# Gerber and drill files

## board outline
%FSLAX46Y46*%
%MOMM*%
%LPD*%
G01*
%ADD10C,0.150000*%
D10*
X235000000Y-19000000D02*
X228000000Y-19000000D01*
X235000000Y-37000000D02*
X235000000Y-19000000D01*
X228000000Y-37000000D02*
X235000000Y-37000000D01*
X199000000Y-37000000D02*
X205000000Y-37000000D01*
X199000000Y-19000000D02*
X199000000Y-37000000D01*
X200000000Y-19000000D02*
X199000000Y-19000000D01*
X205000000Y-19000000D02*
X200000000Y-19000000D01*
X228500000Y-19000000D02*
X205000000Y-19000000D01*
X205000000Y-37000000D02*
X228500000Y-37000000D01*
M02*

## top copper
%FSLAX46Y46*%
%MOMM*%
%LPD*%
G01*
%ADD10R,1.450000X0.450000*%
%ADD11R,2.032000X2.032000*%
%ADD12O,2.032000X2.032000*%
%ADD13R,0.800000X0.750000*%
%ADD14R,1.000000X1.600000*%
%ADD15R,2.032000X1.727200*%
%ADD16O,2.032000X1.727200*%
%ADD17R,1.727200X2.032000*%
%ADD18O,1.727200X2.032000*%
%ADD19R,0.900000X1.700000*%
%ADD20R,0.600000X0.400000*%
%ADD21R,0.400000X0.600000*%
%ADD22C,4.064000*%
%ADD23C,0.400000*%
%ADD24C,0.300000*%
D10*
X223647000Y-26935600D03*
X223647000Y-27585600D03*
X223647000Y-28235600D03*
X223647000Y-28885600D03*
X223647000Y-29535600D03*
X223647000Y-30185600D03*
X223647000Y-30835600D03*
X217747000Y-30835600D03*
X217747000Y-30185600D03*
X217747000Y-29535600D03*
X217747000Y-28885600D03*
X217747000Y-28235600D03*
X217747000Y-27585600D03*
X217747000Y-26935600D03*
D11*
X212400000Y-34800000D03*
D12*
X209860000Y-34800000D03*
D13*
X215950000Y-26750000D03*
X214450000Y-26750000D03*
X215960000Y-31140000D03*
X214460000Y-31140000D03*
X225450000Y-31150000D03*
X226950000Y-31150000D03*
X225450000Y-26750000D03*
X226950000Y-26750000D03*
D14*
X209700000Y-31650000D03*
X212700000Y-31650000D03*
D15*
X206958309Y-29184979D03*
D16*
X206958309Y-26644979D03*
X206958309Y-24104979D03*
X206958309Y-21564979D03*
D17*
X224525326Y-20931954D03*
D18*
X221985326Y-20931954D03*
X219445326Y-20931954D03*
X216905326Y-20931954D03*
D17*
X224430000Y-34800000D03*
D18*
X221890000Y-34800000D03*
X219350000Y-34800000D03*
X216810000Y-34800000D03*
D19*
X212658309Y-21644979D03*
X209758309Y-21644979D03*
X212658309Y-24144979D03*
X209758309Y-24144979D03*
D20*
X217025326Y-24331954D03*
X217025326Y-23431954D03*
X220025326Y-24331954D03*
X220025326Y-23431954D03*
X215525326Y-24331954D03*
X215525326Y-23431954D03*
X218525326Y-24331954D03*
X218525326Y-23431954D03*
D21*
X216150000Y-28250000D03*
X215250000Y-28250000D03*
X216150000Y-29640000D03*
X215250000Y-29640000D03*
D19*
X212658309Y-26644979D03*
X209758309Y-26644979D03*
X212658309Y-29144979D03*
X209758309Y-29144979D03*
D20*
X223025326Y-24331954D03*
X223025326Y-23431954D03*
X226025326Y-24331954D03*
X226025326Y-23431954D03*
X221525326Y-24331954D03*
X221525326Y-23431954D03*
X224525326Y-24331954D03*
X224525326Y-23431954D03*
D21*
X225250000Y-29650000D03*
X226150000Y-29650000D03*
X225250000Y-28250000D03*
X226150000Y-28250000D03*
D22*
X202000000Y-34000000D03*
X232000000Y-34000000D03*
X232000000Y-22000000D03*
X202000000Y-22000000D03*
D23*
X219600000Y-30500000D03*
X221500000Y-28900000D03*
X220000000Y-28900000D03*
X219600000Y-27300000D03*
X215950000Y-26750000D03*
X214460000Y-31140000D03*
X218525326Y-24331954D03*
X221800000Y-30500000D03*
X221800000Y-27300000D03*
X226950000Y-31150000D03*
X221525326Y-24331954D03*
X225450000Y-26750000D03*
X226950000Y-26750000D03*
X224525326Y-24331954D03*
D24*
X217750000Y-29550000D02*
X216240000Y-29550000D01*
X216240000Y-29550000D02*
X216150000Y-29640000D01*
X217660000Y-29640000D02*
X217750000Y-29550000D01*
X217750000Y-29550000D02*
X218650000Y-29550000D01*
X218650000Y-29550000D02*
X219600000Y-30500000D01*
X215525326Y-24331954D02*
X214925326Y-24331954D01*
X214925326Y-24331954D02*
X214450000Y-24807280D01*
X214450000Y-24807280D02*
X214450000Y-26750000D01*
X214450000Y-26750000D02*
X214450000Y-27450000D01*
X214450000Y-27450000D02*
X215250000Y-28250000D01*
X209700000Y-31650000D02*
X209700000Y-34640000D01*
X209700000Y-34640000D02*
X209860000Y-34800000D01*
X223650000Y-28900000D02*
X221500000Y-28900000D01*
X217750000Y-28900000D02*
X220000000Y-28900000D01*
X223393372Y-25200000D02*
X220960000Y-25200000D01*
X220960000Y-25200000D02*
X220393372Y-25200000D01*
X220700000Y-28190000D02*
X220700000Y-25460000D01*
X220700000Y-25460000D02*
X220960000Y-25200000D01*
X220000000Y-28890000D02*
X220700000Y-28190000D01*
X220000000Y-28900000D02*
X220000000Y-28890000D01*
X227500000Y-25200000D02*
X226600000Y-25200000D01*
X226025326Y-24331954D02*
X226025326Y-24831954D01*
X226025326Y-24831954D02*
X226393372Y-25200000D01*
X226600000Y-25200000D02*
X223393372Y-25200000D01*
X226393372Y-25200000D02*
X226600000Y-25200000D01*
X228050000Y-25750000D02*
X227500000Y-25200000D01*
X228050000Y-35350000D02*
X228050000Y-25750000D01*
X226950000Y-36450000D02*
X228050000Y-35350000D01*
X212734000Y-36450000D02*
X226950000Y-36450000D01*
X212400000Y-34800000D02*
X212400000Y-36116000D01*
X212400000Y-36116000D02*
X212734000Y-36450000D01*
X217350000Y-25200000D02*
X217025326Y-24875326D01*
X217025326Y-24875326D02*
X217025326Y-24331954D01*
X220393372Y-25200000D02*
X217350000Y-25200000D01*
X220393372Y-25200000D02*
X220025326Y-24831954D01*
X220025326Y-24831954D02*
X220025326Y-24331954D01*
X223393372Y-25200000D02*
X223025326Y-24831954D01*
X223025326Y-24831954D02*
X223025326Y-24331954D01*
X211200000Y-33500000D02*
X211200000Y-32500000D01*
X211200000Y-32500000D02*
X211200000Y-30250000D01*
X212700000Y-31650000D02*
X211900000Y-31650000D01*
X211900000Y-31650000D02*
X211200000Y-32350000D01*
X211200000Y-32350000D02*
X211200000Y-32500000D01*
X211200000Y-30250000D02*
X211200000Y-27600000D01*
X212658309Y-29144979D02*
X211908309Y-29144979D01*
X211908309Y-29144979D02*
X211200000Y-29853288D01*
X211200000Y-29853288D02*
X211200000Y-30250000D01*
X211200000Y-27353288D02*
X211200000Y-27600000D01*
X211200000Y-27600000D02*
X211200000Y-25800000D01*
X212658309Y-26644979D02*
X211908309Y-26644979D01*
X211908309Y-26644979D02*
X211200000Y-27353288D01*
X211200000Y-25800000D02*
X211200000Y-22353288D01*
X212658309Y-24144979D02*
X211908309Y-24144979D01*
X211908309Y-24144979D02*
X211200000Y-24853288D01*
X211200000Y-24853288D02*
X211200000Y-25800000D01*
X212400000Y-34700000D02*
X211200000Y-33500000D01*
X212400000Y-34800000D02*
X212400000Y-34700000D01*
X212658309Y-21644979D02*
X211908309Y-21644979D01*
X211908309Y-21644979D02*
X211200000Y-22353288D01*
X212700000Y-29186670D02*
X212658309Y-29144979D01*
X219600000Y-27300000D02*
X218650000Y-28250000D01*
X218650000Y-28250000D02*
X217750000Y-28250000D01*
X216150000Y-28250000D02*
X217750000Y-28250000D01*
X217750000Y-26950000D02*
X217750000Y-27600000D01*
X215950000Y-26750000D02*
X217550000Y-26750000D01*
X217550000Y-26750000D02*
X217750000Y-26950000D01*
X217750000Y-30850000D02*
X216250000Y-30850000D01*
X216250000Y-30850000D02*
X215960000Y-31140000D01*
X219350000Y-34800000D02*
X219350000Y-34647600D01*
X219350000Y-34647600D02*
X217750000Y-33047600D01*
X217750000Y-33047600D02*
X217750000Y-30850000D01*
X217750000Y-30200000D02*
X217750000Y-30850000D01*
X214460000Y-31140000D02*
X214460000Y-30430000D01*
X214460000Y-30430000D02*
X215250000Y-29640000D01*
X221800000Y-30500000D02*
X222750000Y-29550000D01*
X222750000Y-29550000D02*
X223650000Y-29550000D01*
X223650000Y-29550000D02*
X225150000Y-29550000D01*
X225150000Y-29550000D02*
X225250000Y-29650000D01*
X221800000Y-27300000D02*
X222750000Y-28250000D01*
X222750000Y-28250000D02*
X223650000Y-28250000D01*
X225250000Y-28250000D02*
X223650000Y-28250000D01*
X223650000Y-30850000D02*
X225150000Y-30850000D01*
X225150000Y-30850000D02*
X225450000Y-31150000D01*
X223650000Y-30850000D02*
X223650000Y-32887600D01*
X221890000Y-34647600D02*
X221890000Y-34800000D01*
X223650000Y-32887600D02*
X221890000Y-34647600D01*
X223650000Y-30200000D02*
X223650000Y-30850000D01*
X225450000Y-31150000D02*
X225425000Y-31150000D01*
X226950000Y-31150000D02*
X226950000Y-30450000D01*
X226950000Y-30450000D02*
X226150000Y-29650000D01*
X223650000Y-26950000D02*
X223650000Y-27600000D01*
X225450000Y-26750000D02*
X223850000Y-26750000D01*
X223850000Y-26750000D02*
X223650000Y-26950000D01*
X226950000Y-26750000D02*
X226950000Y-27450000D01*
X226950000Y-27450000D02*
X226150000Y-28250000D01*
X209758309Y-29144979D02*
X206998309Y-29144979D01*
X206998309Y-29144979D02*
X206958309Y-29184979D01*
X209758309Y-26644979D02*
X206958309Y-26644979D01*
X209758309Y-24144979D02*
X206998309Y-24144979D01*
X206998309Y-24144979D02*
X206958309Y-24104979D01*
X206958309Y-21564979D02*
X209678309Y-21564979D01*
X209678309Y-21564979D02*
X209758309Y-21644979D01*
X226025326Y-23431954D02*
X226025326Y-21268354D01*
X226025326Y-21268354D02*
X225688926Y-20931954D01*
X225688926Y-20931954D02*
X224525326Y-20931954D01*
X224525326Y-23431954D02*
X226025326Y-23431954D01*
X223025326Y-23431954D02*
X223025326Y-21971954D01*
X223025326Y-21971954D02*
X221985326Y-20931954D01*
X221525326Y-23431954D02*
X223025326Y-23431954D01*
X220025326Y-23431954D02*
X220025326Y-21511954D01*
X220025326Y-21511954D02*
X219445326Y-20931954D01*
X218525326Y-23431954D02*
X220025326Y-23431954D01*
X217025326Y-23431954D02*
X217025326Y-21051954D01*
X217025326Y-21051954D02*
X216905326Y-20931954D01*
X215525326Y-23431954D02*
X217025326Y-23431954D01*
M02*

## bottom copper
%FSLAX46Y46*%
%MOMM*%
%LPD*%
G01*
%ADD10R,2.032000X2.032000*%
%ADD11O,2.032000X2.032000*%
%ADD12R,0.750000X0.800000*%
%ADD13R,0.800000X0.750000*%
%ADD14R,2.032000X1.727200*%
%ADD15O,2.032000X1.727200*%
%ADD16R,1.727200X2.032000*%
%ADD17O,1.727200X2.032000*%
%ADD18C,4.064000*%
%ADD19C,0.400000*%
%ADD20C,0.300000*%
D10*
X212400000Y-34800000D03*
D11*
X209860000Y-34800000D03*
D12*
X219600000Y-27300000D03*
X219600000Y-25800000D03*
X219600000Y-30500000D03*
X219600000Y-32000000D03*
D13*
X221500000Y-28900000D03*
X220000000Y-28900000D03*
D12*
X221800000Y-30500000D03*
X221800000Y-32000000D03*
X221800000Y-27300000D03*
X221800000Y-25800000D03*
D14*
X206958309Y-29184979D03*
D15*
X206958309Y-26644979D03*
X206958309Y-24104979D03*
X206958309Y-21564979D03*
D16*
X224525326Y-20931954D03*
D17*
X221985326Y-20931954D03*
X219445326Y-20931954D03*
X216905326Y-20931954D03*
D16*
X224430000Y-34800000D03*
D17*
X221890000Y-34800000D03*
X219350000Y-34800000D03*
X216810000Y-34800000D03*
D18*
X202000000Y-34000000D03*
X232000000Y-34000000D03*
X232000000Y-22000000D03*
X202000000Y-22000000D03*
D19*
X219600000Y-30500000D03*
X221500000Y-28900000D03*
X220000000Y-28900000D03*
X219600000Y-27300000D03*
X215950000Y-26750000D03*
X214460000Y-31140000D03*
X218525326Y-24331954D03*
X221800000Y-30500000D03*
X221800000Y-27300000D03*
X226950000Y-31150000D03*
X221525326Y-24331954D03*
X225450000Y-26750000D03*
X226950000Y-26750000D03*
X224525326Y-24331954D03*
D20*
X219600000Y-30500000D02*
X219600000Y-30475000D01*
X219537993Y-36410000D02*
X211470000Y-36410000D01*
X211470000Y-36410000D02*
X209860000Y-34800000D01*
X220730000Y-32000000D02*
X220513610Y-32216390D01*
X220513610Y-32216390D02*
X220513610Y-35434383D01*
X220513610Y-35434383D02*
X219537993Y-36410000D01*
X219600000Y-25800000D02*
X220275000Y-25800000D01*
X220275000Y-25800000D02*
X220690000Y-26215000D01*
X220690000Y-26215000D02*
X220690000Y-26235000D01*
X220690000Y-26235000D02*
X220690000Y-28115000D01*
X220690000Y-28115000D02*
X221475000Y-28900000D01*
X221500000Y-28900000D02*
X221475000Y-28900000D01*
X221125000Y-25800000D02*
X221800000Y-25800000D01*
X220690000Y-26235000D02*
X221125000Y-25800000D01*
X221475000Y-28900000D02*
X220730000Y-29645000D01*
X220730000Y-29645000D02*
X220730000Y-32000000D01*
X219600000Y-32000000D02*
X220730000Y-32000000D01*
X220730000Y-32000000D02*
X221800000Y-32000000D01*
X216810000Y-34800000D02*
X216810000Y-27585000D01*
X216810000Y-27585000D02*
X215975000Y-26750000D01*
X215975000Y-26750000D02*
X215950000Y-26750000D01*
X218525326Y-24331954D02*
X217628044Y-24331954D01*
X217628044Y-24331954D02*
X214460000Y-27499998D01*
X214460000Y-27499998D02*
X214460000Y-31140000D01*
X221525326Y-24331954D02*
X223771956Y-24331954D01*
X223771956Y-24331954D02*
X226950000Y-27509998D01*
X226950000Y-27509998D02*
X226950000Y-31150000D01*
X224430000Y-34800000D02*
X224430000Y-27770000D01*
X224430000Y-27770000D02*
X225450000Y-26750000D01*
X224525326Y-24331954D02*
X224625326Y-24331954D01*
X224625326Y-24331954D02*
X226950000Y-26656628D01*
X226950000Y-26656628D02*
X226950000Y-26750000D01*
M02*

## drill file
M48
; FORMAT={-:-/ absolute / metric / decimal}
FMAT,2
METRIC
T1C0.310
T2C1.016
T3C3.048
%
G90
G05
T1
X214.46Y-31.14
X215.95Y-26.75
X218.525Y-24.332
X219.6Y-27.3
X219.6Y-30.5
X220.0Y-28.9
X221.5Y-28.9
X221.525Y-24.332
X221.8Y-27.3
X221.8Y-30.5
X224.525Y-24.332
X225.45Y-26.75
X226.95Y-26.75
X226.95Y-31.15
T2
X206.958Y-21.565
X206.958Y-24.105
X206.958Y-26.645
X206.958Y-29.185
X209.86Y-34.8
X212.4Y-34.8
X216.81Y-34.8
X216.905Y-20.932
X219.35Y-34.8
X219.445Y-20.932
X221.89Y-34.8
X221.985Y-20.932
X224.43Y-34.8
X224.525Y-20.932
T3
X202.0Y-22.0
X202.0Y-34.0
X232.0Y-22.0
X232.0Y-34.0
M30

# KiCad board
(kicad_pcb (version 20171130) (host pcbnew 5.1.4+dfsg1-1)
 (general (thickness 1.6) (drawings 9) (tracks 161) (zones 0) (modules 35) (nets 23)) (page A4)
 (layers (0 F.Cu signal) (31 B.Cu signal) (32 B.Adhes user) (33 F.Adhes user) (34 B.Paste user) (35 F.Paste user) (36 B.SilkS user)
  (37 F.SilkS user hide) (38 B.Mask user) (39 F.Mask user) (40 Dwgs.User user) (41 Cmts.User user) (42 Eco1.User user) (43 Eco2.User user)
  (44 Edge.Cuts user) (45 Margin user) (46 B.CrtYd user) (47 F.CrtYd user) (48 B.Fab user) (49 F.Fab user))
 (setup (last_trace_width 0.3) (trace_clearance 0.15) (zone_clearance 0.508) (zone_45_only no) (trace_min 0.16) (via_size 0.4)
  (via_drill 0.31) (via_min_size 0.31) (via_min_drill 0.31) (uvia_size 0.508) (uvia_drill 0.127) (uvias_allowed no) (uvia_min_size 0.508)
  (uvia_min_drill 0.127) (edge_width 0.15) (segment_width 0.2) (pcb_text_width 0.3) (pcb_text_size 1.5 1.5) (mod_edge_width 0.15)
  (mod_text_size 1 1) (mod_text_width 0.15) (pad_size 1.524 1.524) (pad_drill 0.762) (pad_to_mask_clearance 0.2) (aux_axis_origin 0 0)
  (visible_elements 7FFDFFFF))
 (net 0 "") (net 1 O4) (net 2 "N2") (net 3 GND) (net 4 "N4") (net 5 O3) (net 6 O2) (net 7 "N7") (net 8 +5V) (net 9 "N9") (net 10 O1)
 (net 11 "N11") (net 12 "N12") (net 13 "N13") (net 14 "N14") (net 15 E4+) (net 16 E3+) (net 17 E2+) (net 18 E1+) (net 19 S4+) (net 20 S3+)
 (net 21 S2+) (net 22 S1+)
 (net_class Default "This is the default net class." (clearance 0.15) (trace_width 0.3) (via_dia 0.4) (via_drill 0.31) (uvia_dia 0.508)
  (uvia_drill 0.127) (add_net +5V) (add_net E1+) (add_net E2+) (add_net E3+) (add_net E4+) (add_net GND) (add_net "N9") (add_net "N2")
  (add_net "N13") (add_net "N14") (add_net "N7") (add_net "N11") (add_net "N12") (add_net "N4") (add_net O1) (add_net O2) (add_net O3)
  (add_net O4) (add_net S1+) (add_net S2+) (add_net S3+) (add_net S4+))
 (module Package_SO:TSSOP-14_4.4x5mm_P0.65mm (layer F.Cu) (at 220.697 28.8856)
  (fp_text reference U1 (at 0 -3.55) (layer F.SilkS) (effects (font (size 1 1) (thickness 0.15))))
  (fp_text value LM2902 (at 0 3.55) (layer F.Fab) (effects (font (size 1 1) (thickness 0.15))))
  (pad 14 smd rect (at 2.95 -1.95) (size 1.45 0.45) (layers F.Cu F.Paste F.Mask) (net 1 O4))
  (pad 13 smd rect (at 2.95 -1.3) (size 1.45 0.45) (layers F.Cu F.Paste F.Mask) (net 1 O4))
  (pad 12 smd rect (at 2.95 -0.65) (size 1.45 0.45) (layers F.Cu F.Paste F.Mask) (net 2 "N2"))
  (pad 11 smd rect (at 2.95 0) (size 1.45 0.45) (layers F.Cu F.Paste F.Mask) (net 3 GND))
  (pad 10 smd rect (at 2.95 0.65) (size 1.45 0.45) (layers F.Cu F.Paste F.Mask) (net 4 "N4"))
  (pad 9 smd rect (at 2.95 1.3) (size 1.45 0.45) (layers F.Cu F.Paste F.Mask) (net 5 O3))
  (pad 8 smd rect (at 2.95 1.95) (size 1.45 0.45) (layers F.Cu F.Paste F.Mask) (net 5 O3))
  (pad 7 smd rect (at -2.95 1.95) (size 1.45 0.45) (layers F.Cu F.Paste F.Mask) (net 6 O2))
  (pad 6 smd rect (at -2.95 1.3) (size 1.45 0.45) (layers F.Cu F.Paste F.Mask) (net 6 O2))
  (pad 5 smd rect (at -2.95 0.65) (size 1.45 0.45) (layers F.Cu F.Paste F.Mask) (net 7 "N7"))
  (pad 4 smd rect (at -2.95 0) (size 1.45 0.45) (layers F.Cu F.Paste F.Mask) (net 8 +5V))
  (pad 3 smd rect (at -2.95 -0.65) (size 1.45 0.45) (layers F.Cu F.Paste F.Mask) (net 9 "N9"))
  (pad 2 smd rect (at -2.95 -1.3) (size 1.45 0.45) (layers F.Cu F.Paste F.Mask) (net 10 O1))
  (pad 1 smd rect (at -2.95 -1.95) (size 1.45 0.45) (layers F.Cu F.Paste F.Mask) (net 10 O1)))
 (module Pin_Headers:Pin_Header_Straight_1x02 (layer F.Cu) (at 212.4 34.8 270)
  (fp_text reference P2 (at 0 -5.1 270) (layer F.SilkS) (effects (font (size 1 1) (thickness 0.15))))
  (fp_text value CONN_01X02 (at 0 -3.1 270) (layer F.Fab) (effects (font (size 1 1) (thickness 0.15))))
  (pad 1 thru_hole rect (at 0 0 270) (size 2.032 2.032) (drill 1.016) (layers *.Cu *.Mask F.SilkS) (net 8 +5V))
  (pad 2 thru_hole oval (at 0 2.54 270) (size 2.032 2.032) (drill 1.016) (layers *.Cu *.Mask F.SilkS) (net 3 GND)))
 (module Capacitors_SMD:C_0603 (layer B.Cu) (at 219.6 26.55 90)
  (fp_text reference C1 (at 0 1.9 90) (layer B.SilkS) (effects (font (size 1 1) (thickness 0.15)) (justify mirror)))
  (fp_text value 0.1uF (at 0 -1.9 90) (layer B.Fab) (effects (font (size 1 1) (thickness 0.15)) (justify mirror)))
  (pad 1 smd rect (at -0.75 0 90) (size 0.8 0.75) (layers B.Cu B.Paste B.Mask) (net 9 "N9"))
  (pad 2 smd rect (at 0.75 0 90) (size 0.8 0.75) (layers B.Cu B.Paste B.Mask) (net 3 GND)))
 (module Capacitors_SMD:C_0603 (layer B.Cu) (at 219.6 31.25 270)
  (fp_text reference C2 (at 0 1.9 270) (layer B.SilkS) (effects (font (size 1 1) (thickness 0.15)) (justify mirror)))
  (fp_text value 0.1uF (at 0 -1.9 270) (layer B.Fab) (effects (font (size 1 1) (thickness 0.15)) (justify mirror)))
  (pad 1 smd rect (at -0.75 0 270) (size 0.8 0.75) (layers B.Cu B.Paste B.Mask) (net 7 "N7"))
  (pad 2 smd rect (at 0.75 0 270) (size 0.8 0.75) (layers B.Cu B.Paste B.Mask) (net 3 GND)))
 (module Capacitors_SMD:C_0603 (layer F.Cu) (at 215.2 26.75 180)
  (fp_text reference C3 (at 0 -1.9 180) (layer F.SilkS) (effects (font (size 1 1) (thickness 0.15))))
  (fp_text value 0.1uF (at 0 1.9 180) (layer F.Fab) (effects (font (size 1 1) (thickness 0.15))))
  (pad 1 smd rect (at -0.75 0 180) (size 0.8 0.75) (layers F.Cu F.Paste F.Mask) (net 10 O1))
  (pad 2 smd rect (at 0.75 0 180) (size 0.8 0.75) (layers F.Cu F.Paste F.Mask) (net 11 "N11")))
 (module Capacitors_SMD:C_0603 (layer F.Cu) (at 215.21 31.14 180)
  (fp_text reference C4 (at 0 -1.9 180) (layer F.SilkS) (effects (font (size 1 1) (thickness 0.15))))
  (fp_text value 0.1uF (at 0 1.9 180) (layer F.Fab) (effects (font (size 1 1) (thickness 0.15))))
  (pad 1 smd rect (at -0.75 0 180) (size 0.8 0.75) (layers F.Cu F.Paste F.Mask) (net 6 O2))
  (pad 2 smd rect (at 0.75 0 180) (size 0.8 0.75) (layers F.Cu F.Paste F.Mask) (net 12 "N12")))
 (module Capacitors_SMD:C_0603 (layer B.Cu) (at 220.75 28.9 180)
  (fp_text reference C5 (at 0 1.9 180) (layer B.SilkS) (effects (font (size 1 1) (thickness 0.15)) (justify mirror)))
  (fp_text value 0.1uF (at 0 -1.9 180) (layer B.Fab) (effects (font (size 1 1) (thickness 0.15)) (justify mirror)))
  (pad 1 smd rect (at -0.75 0 180) (size 0.8 0.75) (layers B.Cu B.Paste B.Mask) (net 3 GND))
  (pad 2 smd rect (at 0.75 0 180) (size 0.8 0.75) (layers B.Cu B.Paste B.Mask) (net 8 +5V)))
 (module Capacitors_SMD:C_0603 (layer B.Cu) (at 221.8 31.25 270)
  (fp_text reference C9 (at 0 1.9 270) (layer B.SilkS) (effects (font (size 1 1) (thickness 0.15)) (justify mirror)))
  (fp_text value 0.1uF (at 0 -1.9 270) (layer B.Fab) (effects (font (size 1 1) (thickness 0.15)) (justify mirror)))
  (pad 1 smd rect (at -0.75 0 270) (size 0.8 0.75) (layers B.Cu B.Paste B.Mask) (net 4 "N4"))
  (pad 2 smd rect (at 0.75 0 270) (size 0.8 0.75) (layers B.Cu B.Paste B.Mask) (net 3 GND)))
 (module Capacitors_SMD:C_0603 (layer B.Cu) (at 221.8 26.55 90)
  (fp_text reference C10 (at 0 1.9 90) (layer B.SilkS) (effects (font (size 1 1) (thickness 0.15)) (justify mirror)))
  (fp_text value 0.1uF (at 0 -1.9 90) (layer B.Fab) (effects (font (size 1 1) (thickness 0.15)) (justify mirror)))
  (pad 1 smd rect (at -0.75 0 90) (size 0.8 0.75) (layers B.Cu B.Paste B.Mask) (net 2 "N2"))
  (pad 2 smd rect (at 0.75 0 90) (size 0.8 0.75) (layers B.Cu B.Paste B.Mask) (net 3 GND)))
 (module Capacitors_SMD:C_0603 (layer F.Cu) (at 226.2 31.15)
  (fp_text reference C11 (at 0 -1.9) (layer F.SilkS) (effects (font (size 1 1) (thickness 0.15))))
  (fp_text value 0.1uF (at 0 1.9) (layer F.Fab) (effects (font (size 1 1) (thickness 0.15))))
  (pad 1 smd rect (at -0.75 0) (size 0.8 0.75) (layers F.Cu F.Paste F.Mask) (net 5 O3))
  (pad 2 smd rect (at 0.75 0) (size 0.8 0.75) (layers F.Cu F.Paste F.Mask) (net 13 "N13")))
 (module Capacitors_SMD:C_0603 (layer F.Cu) (at 226.2 26.75)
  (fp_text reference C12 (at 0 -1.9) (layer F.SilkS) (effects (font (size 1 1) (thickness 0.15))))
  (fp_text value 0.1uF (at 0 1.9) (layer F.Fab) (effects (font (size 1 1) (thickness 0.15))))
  (pad 1 smd rect (at -0.75 0) (size 0.8 0.75) (layers F.Cu F.Paste F.Mask) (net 1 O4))
  (pad 2 smd rect (at 0.75 0) (size 0.8 0.75) (layers F.Cu F.Paste F.Mask) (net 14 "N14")))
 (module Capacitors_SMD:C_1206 (layer F.Cu) (at 211.2 31.65)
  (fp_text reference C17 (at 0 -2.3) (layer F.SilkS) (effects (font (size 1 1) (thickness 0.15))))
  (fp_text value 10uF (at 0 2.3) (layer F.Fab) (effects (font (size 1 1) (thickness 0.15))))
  (pad 1 smd rect (at -1.5 0) (size 1 1.6) (layers F.Cu F.Paste F.Mask) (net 3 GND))
  (pad 2 smd rect (at 1.5 0) (size 1 1.6) (layers F.Cu F.Paste F.Mask) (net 8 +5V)))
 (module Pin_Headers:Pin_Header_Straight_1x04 (layer F.Cu) (at 206.958309 29.184979 180)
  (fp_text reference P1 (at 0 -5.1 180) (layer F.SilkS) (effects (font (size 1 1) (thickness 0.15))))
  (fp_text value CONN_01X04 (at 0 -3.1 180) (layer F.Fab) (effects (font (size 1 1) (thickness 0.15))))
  (pad 1 thru_hole rect (at 0 0 180) (size 2.032 1.7272) (drill 1.016) (layers *.Cu *.Mask F.SilkS) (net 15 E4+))
  (pad 2 thru_hole oval (at 0 2.54 180) (size 2.032 1.7272) (drill 1.016) (layers *.Cu *.Mask F.SilkS) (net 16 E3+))
  (pad 3 thru_hole oval (at 0 5.08 180) (size 2.032 1.7272) (drill 1.016) (layers *.Cu *.Mask F.SilkS) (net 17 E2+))
  (pad 4 thru_hole oval (at 0 7.62 180) (size 2.032 1.7272) (drill 1.016) (layers *.Cu *.Mask F.SilkS) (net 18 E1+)))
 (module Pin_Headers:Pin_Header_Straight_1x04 (layer F.Cu) (at 224.525326 20.931954 270)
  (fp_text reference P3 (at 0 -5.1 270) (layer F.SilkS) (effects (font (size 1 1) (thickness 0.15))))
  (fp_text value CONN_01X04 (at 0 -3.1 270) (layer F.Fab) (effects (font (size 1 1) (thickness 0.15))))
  (pad 1 thru_hole rect (at 0 0 270) (size 2.032 1.7272) (drill 1.016) (layers *.Cu *.Mask F.SilkS) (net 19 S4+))
  (pad 2 thru_hole oval (at 0 2.54 270) (size 2.032 1.7272) (drill 1.016) (layers *.Cu *.Mask F.SilkS) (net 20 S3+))
  (pad 3 thru_hole oval (at 0 5.08 270) (size 2.032 1.7272) (drill 1.016) (layers *.Cu *.Mask F.SilkS) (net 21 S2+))
  (pad 4 thru_hole oval (at 0 7.62 270) (size 2.032 1.7272) (drill 1.016) (layers *.Cu *.Mask F.SilkS) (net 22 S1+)))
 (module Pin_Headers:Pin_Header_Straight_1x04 (layer F.Cu) (at 224.43 34.8 270)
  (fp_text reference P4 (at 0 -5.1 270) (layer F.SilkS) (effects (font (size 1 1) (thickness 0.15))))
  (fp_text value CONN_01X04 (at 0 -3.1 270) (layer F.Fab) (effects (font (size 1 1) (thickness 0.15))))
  (pad 1 thru_hole rect (at 0 0 270) (size 2.032 1.7272) (drill 1.016) (layers *.Cu *.Mask F.SilkS) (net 1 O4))
  (pad 2 thru_hole oval (at 0 2.54 270) (size 2.032 1.7272) (drill 1.016) (layers *.Cu *.Mask F.SilkS) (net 5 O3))
  (pad 3 thru_hole oval (at 0 5.08 270) (size 2.032 1.7272) (drill 1.016) (layers *.Cu *.Mask F.SilkS) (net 6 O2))
  (pad 4 thru_hole oval (at 0 7.62 270) (size 2.032 1.7272) (drill 1.016) (layers *.Cu *.Mask F.SilkS) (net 10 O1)))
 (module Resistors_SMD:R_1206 (layer F.Cu) (at 211.208309 21.644979 180)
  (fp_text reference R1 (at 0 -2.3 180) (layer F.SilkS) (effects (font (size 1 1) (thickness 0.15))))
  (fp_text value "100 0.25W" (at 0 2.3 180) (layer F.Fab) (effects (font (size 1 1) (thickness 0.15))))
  (pad 1 smd rect (at -1.45 0 180) (size 0.9 1.7) (layers F.Cu F.Paste F.Mask) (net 8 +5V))
  (pad 2 smd rect (at 1.45 0 180) (size 0.9 1.7) (layers F.Cu F.Paste F.Mask) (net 18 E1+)))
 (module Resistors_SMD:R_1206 (layer F.Cu) (at 211.208309 24.144979 180)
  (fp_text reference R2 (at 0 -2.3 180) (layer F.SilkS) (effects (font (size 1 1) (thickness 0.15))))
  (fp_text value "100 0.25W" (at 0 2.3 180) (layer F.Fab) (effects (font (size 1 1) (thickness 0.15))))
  (pad 1 smd rect (at -1.45 0 180) (size 0.9 1.7) (layers F.Cu F.Paste F.Mask) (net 8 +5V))
  (pad 2 smd rect (at 1.45 0 180) (size 0.9 1.7) (layers F.Cu F.Paste F.Mask) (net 17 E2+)))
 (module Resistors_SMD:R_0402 (layer F.Cu) (at 217.025326 23.881954 90)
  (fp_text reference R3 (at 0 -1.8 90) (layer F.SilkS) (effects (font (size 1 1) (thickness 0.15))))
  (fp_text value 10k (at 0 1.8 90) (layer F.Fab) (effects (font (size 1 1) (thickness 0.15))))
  (pad 1 smd rect (at -0.45 0 90) (size 0.4 0.6) (layers F.Cu F.Paste F.Mask) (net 8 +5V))
  (pad 2 smd rect (at 0.45 0 90) (size 0.4 0.6) (layers F.Cu F.Paste F.Mask) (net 22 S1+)))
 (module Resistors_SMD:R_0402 (layer F.Cu) (at 220.025326 23.881954 90)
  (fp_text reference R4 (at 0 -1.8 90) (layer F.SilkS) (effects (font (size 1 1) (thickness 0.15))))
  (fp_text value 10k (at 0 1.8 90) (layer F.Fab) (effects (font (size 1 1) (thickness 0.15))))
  (pad 1 smd rect (at -0.45 0 90) (size 0.4 0.6) (layers F.Cu F.Paste F.Mask) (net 8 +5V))
  (pad 2 smd rect (at 0.45 0 90) (size 0.4 0.6) (layers F.Cu F.Paste F.Mask) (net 21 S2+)))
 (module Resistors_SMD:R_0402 (layer F.Cu) (at 215.525326 23.881954 90)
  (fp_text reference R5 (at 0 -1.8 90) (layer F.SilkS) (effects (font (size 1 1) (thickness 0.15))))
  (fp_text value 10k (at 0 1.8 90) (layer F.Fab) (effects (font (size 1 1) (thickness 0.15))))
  (pad 1 smd rect (at -0.45 0 90) (size 0.4 0.6) (layers F.Cu F.Paste F.Mask) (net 11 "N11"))
  (pad 2 smd rect (at 0.45 0 90) (size 0.4 0.6) (layers F.Cu F.Paste F.Mask) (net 22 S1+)))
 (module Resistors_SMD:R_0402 (layer F.Cu) (at 218.525326 23.881954 90)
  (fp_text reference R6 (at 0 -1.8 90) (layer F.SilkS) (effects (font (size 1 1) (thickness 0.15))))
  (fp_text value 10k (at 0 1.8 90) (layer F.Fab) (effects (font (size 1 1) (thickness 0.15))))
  (pad 1 smd rect (at -0.45 0 90) (size 0.4 0.6) (layers F.Cu F.Paste F.Mask) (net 12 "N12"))
  (pad 2 smd rect (at 0.45 0 90) (size 0.4 0.6) (layers F.Cu F.Paste F.Mask) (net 21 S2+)))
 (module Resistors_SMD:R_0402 (layer F.Cu) (at 215.7 28.25 180)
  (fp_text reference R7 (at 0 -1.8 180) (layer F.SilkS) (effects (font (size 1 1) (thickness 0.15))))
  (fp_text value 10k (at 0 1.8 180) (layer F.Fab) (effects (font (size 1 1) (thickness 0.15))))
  (pad 1 smd rect (at -0.45 0 180) (size 0.4 0.6) (layers F.Cu F.Paste F.Mask) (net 9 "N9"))
  (pad 2 smd rect (at 0.45 0 180) (size 0.4 0.6) (layers F.Cu F.Paste F.Mask) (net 11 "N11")))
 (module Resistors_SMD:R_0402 (layer F.Cu) (at 215.7 29.64 180)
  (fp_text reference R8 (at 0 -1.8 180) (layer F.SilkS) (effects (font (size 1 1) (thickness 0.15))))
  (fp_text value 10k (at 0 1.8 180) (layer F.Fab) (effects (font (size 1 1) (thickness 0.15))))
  (pad 1 smd rect (at -0.45 0 180) (size 0.4 0.6) (layers F.Cu F.Paste F.Mask) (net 7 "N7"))
  (pad 2 smd rect (at 0.45 0 180) (size 0.4 0.6) (layers F.Cu F.Paste F.Mask) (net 12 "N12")))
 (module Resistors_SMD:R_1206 (layer F.Cu) (at 211.208309 26.644979 180)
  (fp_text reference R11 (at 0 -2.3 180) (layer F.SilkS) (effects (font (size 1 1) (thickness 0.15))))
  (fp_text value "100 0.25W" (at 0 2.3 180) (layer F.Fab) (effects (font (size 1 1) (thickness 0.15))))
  (pad 1 smd rect (at -1.45 0 180) (size 0.9 1.7) (layers F.Cu F.Paste F.Mask) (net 8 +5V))
  (pad 2 smd rect (at 1.45 0 180) (size 0.9 1.7) (layers F.Cu F.Paste F.Mask) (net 16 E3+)))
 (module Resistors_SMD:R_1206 (layer F.Cu) (at 211.208309 29.144979 180)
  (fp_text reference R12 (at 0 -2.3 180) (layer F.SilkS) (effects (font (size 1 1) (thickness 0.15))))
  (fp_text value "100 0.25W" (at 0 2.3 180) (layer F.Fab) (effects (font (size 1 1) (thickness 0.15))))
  (pad 1 smd rect (at -1.45 0 180) (size 0.9 1.7) (layers F.Cu F.Paste F.Mask) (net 8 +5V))
  (pad 2 smd rect (at 1.45 0 180) (size 0.9 1.7) (layers F.Cu F.Paste F.Mask) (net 15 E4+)))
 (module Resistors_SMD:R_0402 (layer F.Cu) (at 223.025326 23.881954 90)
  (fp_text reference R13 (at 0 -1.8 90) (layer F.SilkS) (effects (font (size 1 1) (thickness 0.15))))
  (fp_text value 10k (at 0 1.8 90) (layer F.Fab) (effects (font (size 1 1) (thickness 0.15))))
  (pad 1 smd rect (at -0.45 0 90) (size 0.4 0.6) (layers F.Cu F.Paste F.Mask) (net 8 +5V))
  (pad 2 smd rect (at 0.45 0 90) (size 0.4 0.6) (layers F.Cu F.Paste F.Mask) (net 20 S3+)))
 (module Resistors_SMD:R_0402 (layer F.Cu) (at 226.025326 23.881954 90)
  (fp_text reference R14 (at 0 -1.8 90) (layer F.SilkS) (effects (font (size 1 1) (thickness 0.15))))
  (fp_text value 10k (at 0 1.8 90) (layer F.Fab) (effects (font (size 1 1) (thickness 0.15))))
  (pad 1 smd rect (at -0.45 0 90) (size 0.4 0.6) (layers F.Cu F.Paste F.Mask) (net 8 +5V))
  (pad 2 smd rect (at 0.45 0 90) (size 0.4 0.6) (layers F.Cu F.Paste F.Mask) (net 19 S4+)))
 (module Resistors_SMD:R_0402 (layer F.Cu) (at 221.525326 23.881954 90)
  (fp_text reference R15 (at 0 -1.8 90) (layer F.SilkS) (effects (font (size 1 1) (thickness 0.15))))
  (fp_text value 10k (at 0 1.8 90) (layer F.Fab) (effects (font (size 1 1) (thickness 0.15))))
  (pad 1 smd rect (at -0.45 0 90) (size 0.4 0.6) (layers F.Cu F.Paste F.Mask) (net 13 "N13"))
  (pad 2 smd rect (at 0.45 0 90) (size 0.4 0.6) (layers F.Cu F.Paste F.Mask) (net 20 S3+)))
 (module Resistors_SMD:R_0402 (layer F.Cu) (at 224.525326 23.881954 90)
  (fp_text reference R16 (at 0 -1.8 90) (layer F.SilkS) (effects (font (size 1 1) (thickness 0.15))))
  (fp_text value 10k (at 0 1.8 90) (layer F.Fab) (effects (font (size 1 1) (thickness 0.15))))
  (pad 1 smd rect (at -0.45 0 90) (size 0.4 0.6) (layers F.Cu F.Paste F.Mask) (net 14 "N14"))
  (pad 2 smd rect (at 0.45 0 90) (size 0.4 0.6) (layers F.Cu F.Paste F.Mask) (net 19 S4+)))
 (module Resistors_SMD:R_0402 (layer F.Cu) (at 225.7 29.65)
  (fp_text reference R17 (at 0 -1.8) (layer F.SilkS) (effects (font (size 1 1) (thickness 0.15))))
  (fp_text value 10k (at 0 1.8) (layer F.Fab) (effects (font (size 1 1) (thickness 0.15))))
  (pad 1 smd rect (at -0.45 0) (size 0.4 0.6) (layers F.Cu F.Paste F.Mask) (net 4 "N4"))
  (pad 2 smd rect (at 0.45 0) (size 0.4 0.6) (layers F.Cu F.Paste F.Mask) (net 13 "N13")))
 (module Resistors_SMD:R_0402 (layer F.Cu) (at 225.7 28.25)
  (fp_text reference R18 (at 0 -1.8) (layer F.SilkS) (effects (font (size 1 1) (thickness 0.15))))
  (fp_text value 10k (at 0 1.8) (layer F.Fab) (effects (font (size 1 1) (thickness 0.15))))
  (pad 1 smd rect (at -0.45 0) (size 0.4 0.6) (layers F.Cu F.Paste F.Mask) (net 2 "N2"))
  (pad 2 smd rect (at 0.45 0) (size 0.4 0.6) (layers F.Cu F.Paste F.Mask) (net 14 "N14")))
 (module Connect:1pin (layer F.Cu) (at 202 34)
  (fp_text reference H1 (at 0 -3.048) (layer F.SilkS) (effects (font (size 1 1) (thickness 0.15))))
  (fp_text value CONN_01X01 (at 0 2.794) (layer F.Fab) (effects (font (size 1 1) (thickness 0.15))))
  (pad 1 thru_hole circle (at 0 0) (size 4.064 4.064) (drill 3.048) (layers *.Cu *.Mask F.SilkS)))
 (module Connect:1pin (layer F.Cu) (at 232 34)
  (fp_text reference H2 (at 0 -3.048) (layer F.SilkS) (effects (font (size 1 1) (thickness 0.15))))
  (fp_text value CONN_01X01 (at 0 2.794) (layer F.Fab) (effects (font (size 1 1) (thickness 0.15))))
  (pad 1 thru_hole circle (at 0 0) (size 4.064 4.064) (drill 3.048) (layers *.Cu *.Mask F.SilkS)))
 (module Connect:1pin (layer F.Cu) (at 232 22)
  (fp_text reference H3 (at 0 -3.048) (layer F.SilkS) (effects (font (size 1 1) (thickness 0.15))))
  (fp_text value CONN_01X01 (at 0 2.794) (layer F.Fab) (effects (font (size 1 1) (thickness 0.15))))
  (pad 1 thru_hole circle (at 0 0) (size 4.064 4.064) (drill 3.048) (layers *.Cu *.Mask F.SilkS)))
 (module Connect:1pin (layer F.Cu) (at 202 22)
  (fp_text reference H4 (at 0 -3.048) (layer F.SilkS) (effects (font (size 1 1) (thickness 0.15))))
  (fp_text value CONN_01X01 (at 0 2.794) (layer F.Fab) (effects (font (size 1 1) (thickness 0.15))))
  (pad 1 thru_hole circle (at 0 0) (size 4.064 4.064) (drill 3.048) (layers *.Cu *.Mask F.SilkS)))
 (gr_line (start 235 19) (end 228 19) (layer Edge.Cuts) (width 0.15))
 (gr_line (start 235 37) (end 235 19) (layer Edge.Cuts) (width 0.15))
 (gr_line (start 228 37) (end 235 37) (layer Edge.Cuts) (width 0.15))
 (gr_line (start 199 37) (end 205 37) (layer Edge.Cuts) (width 0.15))
 (gr_line (start 199 19) (end 199 37) (layer Edge.Cuts) (width 0.15))
 (gr_line (start 200 19) (end 199 19) (layer Edge.Cuts) (width 0.15))
 (gr_line (start 205 19) (end 200 19) (layer Edge.Cuts) (width 0.15))
 (gr_line (start 228.5 19) (end 205 19) (layer Edge.Cuts) (width 0.15))
 (gr_line (start 205 37) (end 228.5 37) (layer Edge.Cuts) (width 0.15))
 (segment (start 217.75 29.55) (end 216.24 29.55) (width 0.3) (layer F.Cu) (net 7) (status 30))
 (segment (start 216.24 29.55) (end 216.15 29.64) (width 0.3) (layer F.Cu) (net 7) (status 30))
 (segment (start 217.66 29.64) (end 217.75 29.55) (width 0.3) (layer F.Cu) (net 7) (status 30))
 (segment (start 217.75 29.55) (end 218.65 29.55) (width 0.3) (layer F.Cu) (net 7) (status 10))
 (segment (start 218.65 29.55) (end 219.6 30.5) (width 0.3) (layer F.Cu) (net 7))
 (via (at 219.6 30.5) (size 0.4) (drill 0.31) (layers F.Cu B.Cu) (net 7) (status 30))
 (segment (start 219.6 30.5) (end 219.6 30.475) (width 0.3) (layer B.Cu) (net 7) (status 30))
 (segment (start 215.525326 24.331954) (end 214.925326 24.331954) (width 0.3) (layer F.Cu) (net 11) (status 10))
 (segment (start 214.925326 24.331954) (end 214.45 24.80728) (width 0.3) (layer F.Cu) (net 11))
 (segment (start 214.45 24.80728) (end 214.45 26.75) (width 0.3) (layer F.Cu) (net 11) (status 20))
 (segment (start 214.45 26.75) (end 214.45 27.45) (width 0.3) (layer F.Cu) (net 11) (status 10))
 (segment (start 214.45 27.45) (end 215.25 28.25) (width 0.3) (layer F.Cu) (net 11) (status 20))
 (segment (start 209.7 31.65) (end 209.7 34.64) (width 0.3) (layer F.Cu) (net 3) (status 30))
 (segment (start 209.7 34.64) (end 209.86 34.8) (width 0.3) (layer F.Cu) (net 3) (status 30))
 (segment (start 219.537993 36.41) (end 211.47 36.41) (width 0.3) (layer B.Cu) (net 3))
 (segment (start 211.47 36.41) (end 209.86 34.8) (width 0.3) (layer B.Cu) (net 3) (status 20))
 (segment (start 220.73 32) (end 220.51361 32.21639) (width 0.3) (layer B.Cu) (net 3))
 (segment (start 220.51361 32.21639) (end 220.51361 35.434383) (width 0.3) (layer B.Cu) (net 3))
 (segment (start 220.51361 35.434383) (end 219.537993 36.41) (width 0.3) (layer B.Cu) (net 3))
 (segment (start 219.6 25.8) (end 220.275 25.8) (width 0.3) (layer B.Cu) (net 3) (status 10))
 (segment (start 220.275 25.8) (end 220.69 26.215) (width 0.3) (layer B.Cu) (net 3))
 (segment (start 220.69 26.215) (end 220.69 26.235) (width 0.3) (layer B.Cu) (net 3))
 (segment (start 220.69 26.235) (end 220.69 28.115) (width 0.3) (layer B.Cu) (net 3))
 (segment (start 220.69 28.115) (end 221.475 28.9) (width 0.3) (layer B.Cu) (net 3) (status 20))
 (segment (start 221.5 28.9) (end 221.475 28.9) (width 0.3) (layer B.Cu) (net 3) (status 30))
 (segment (start 221.125 25.8) (end 221.8 25.8) (width 0.3) (layer B.Cu) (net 3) (status 20))
 (segment (start 220.69 26.235) (end 221.125 25.8) (width 0.3) (layer B.Cu) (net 3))
 (segment (start 221.475 28.9) (end 220.73 29.645) (width 0.3) (layer B.Cu) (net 3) (status 10))
 (segment (start 220.73 29.645) (end 220.73 32) (width 0.3) (layer B.Cu) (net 3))
 (segment (start 223.65 28.9) (end 221.5 28.9) (width 0.3) (layer F.Cu) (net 3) (status 10))
 (via (at 221.5 28.9) (size 0.4) (drill 0.31) (layers F.Cu B.Cu) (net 3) (status 30))
 (segment (start 219.6 32) (end 220.73 32) (width 0.3) (layer B.Cu) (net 3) (status 1000010))
 (segment (start 220.73 32) (end 221.8 32) (width 0.3) (layer B.Cu) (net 3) (status 1000020))
 (segment (start 217.75 28.9) (end 220 28.9) (width 0.3) (layer F.Cu) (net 8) (status 10))
 (segment (start 223.393372 25.2) (end 220.96 25.2) (width 0.3) (layer F.Cu) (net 8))
 (segment (start 220.96 25.2) (end 220.393372 25.2) (width 0.3) (layer F.Cu) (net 8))
 (segment (start 220.7 28.19) (end 220.7 25.46) (width 0.3) (layer F.Cu) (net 8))
 (segment (start 220.7 25.46) (end 220.96 25.2) (width 0.3) (layer F.Cu) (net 8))
 (segment (start 220 28.89) (end 220.7 28.19) (width 0.3) (layer F.Cu) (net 8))
 (segment (start 220 28.9) (end 220 28.89) (width 0.3) (layer F.Cu) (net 8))
 (via (at 220 28.9) (size 0.4) (drill 0.31) (layers F.Cu B.Cu) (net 8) (status 30))
 (segment (start 227.5 25.2) (end 226.6 25.2) (width 0.3) (layer F.Cu) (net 8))
 (segment (start 226.025326 24.331954) (end 226.025326 24.831954) (width 0.3) (layer F.Cu) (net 8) (status 10))
 (segment (start 226.025326 24.831954) (end 226.393372 25.2) (width 0.3) (layer F.Cu) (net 8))
 (segment (start 226.6 25.2) (end 223.393372 25.2) (width 0.3) (layer F.Cu) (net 8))
 (segment (start 226.393372 25.2) (end 226.6 25.2) (width 0.3) (layer F.Cu) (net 8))
 (segment (start 228.05 25.75) (end 227.5 25.2) (width 0.3) (layer F.Cu) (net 8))
 (segment (start 228.05 35.35) (end 228.05 25.75) (width 0.3) (layer F.Cu) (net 8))
 (segment (start 226.95 36.45) (end 228.05 35.35) (width 0.3) (layer F.Cu) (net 8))
 (segment (start 212.734 36.45) (end 226.95 36.45) (width 0.3) (layer F.Cu) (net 8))
 (segment (start 212.4 34.8) (end 212.4 36.116) (width 0.3) (layer F.Cu) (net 8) (status 10))
 (segment (start 212.4 36.116) (end 212.734 36.45) (width 0.3) (layer F.Cu) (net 8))
 (segment (start 217.35 25.2) (end 217.025326 24.875326) (width 0.3) (layer F.Cu) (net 8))
 (segment (start 217.025326 24.875326) (end 217.025326 24.331954) (width 0.3) (layer F.Cu) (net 8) (status 20))
 (segment (start 220.393372 25.2) (end 217.35 25.2) (width 0.3) (layer F.Cu) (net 8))
 (segment (start 220.393372 25.2) (end 220.025326 24.831954) (width 0.3) (layer F.Cu) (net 8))
 (segment (start 220.025326 24.831954) (end 220.025326 24.331954) (width 0.3) (layer F.Cu) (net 8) (status 20))
 (segment (start 223.393372 25.2) (end 223.025326 24.831954) (width 0.3) (layer F.Cu) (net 8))
 (segment (start 223.025326 24.831954) (end 223.025326 24.331954) (width 0.3) (layer F.Cu) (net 8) (status 20))
 (segment (start 211.2 33.5) (end 211.2 32.5) (width 0.3) (layer F.Cu) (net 8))
 (segment (start 211.2 32.5) (end 211.2 30.25) (width 0.3) (layer F.Cu) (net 8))
 (segment (start 212.7 31.65) (end 211.9 31.65) (width 0.3) (layer F.Cu) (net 8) (status 10))
 (segment (start 211.9 31.65) (end 211.2 32.35) (width 0.3) (layer F.Cu) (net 8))
 (segment (start 211.2 32.35) (end 211.2 32.5) (width 0.3) (layer F.Cu) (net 8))
 (segment (start 211.2 30.25) (end 211.2 27.6) (width 0.3) (layer F.Cu) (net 8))
 (segment (start 212.658309 29.144979) (end 211.908309 29.144979) (width 0.3) (layer F.Cu) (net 8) (status 10))
 (segment (start 211.908309 29.144979) (end 211.2 29.853288) (width 0.3) (layer F.Cu) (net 8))
 (segment (start 211.2 29.853288) (end 211.2 30.25) (width 0.3) (layer F.Cu) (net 8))
 (segment (start 211.2 27.353288) (end 211.2 27.6) (width 0.3) (layer F.Cu) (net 8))
 (segment (start 211.2 27.6) (end 211.2 25.8) (width 0.3) (layer F.Cu) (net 8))
 (segment (start 212.658309 26.644979) (end 211.908309 26.644979) (width 0.3) (layer F.Cu) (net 8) (status 10))
 (segment (start 211.908309 26.644979) (end 211.2 27.353288) (width 0.3) (layer F.Cu) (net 8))
 (segment (start 211.2 25.8) (end 211.2 22.353288) (width 0.3) (layer F.Cu) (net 8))
 (segment (start 212.658309 24.144979) (end 211.908309 24.144979) (width 0.3) (layer F.Cu) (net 8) (status 10))
 (segment (start 211.908309 24.144979) (end 211.2 24.853288) (width 0.3) (layer F.Cu) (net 8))
 (segment (start 211.2 24.853288) (end 211.2 25.8) (width 0.3) (layer F.Cu) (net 8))
 (segment (start 212.4 34.7) (end 211.2 33.5) (width 0.3) (layer F.Cu) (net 8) (status 10))
 (segment (start 212.4 34.8) (end 212.4 34.7) (width 0.3) (layer F.Cu) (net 8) (status 30))
 (segment (start 212.658309 21.644979) (end 211.908309 21.644979) (width 0.3) (layer F.Cu) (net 8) (status 10))
 (segment (start 211.908309 21.644979) (end 211.2 22.353288) (width 0.3) (layer F.Cu) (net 8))
 (segment (start 212.7 29.18667) (end 212.658309 29.144979) (width 0.3) (layer F.Cu) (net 8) (status 30))
 (segment (start 219.6 27.3) (end 218.65 28.25) (width 0.3) (layer F.Cu) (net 9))
 (segment (start 218.65 28.25) (end 217.75 28.25) (width 0.3) (layer F.Cu) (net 9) (status 20))
 (segment (start 216.15 28.25) (end 217.75 28.25) (width 0.3) (layer F.Cu) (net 9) (status 30))
 (via (at 219.6 27.3) (size 0.4) (drill 0.31) (layers F.Cu B.Cu) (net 9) (status 30))
 (segment (start 216.81 34.8) (end 216.81 27.585) (width 0.3) (layer B.Cu) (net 10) (status 10))
 (segment (start 216.81 27.585) (end 215.975 26.75) (width 0.3) (layer B.Cu) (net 10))
 (segment (start 215.975 26.75) (end 215.95 26.75) (width 0.3) (layer B.Cu) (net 10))
 (via (at 215.95 26.75) (size 0.4) (drill 0.31) (layers F.Cu B.Cu) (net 10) (status 30))
 (segment (start 217.75 26.95) (end 217.75 27.6) (width 0.3) (layer F.Cu) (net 10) (status 30))
 (segment (start 215.95 26.75) (end 217.55 26.75) (width 0.3) (layer F.Cu) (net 10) (status 30))
 (segment (start 217.55 26.75) (end 217.75 26.95) (width 0.3) (layer F.Cu) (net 10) (status 30))
 (segment (start 217.75 30.85) (end 216.25 30.85) (width 0.3) (layer F.Cu) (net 6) (status 30))
 (segment (start 216.25 30.85) (end 215.96 31.14) (width 0.3) (layer F.Cu) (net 6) (status 30))
 (segment (start 219.35 34.8) (end 219.35 34.6476) (width 0.3) (layer F.Cu) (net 6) (status 30))
 (segment (start 219.35 34.6476) (end 217.75 33.0476) (width 0.3) (layer F.Cu) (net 6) (status 10))
 (segment (start 217.75 33.0476) (end 217.75 30.85) (width 0.3) (layer F.Cu) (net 6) (status 20))
 (segment (start 217.75 30.2) (end 217.75 30.85) (width 0.3) (layer F.Cu) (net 6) (status 30))
 (segment (start 218.525326 24.331954) (end 217.628044 24.331954) (width 0.3) (layer B.Cu) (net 12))
 (segment (start 217.628044 24.331954) (end 214.46 27.499998) (width 0.3) (layer B.Cu) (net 12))
 (segment (start 214.46 27.499998) (end 214.46 31.14) (width 0.3) (layer B.Cu) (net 12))
 (via (at 214.46 31.14) (size 0.4) (drill 0.31) (layers F.Cu B.Cu) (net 12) (status 30))
 (via (at 218.525326 24.331954) (size 0.4) (drill 0.31) (layers F.Cu B.Cu) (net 12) (status 30))
 (segment (start 214.46 31.14) (end 214.46 30.43) (width 0.3) (layer F.Cu) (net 12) (status 10))
 (segment (start 214.46 30.43) (end 215.25 29.64) (width 0.3) (layer F.Cu) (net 12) (status 20))
 (segment (start 221.8 30.5) (end 222.75 29.55) (width 0.3) (layer F.Cu) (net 4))
 (segment (start 222.75 29.55) (end 223.65 29.55) (width 0.3) (layer F.Cu) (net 4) (status 20))
 (segment (start 223.65 29.55) (end 225.15 29.55) (width 0.3) (layer F.Cu) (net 4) (status 30))
 (segment (start 225.15 29.55) (end 225.25 29.65) (width 0.3) (layer F.Cu) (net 4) (status 30))
 (via (at 221.8 30.5) (size 0.4) (drill 0.31) (layers F.Cu B.Cu) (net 4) (status 30))
 (segment (start 221.8 27.3) (end 222.75 28.25) (width 0.3) (layer F.Cu) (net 2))
 (segment (start 222.75 28.25) (end 223.65 28.25) (width 0.3) (layer F.Cu) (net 2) (status 20))
 (segment (start 225.25 28.25) (end 223.65 28.25) (width 0.3) (layer F.Cu) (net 2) (status 30))
 (via (at 221.8 27.3) (size 0.4) (drill 0.31) (layers F.Cu B.Cu) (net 2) (status 30))
 (segment (start 223.65 30.85) (end 225.15 30.85) (width 0.3) (layer F.Cu) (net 5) (status 30))
 (segment (start 225.15 30.85) (end 225.45 31.15) (width 0.3) (layer F.Cu) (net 5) (status 30))
 (segment (start 223.65 30.85) (end 223.65 32.8876) (width 0.3) (layer F.Cu) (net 5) (status 10))
 (segment (start 221.89 34.6476) (end 221.89 34.8) (width 0.3) (layer F.Cu) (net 5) (status 30))
 (segment (start 223.65 32.8876) (end 221.89 34.6476) (width 0.3) (layer F.Cu) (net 5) (status 20))
 (segment (start 223.65 30.2) (end 223.65 30.85) (width 0.3) (layer F.Cu) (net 5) (status 30))
 (segment (start 225.45 31.15) (end 225.425 31.15) (width 0.3) (layer F.Cu) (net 5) (status 30))
 (segment (start 221.525326 24.331954) (end 223.771956 24.331954) (width 0.3) (layer B.Cu) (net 13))
 (segment (start 223.771956 24.331954) (end 226.95 27.509998) (width 0.3) (layer B.Cu) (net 13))
 (segment (start 226.95 27.509998) (end 226.95 31.15) (width 0.3) (layer B.Cu) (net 13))
 (via (at 226.95 31.15) (size 0.4) (drill 0.31) (layers F.Cu B.Cu) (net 13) (status 30))
 (segment (start 226.95 31.15) (end 226.95 30.45) (width 0.3) (layer F.Cu) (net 13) (status 10))
 (segment (start 226.95 30.45) (end 226.15 29.65) (width 0.3) (layer F.Cu) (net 13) (status 20))
 (via (at 221.525326 24.331954) (size 0.4) (drill 0.31) (layers F.Cu B.Cu) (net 13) (status 30))
 (segment (start 223.65 26.95) (end 223.65 27.6) (width 0.3) (layer F.Cu) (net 1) (status 30))
 (segment (start 224.43 34.8) (end 224.43 27.77) (width 0.3) (layer B.Cu) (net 1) (status 10))
 (segment (start 224.43 27.77) (end 225.45 26.75) (width 0.3) (layer B.Cu) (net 1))
 (via (at 225.45 26.75) (size 0.4) (drill 0.31) (layers F.Cu B.Cu) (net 1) (status 30))
 (segment (start 225.45 26.75) (end 223.85 26.75) (width 0.3) (layer F.Cu) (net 1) (status 30))
 (segment (start 223.85 26.75) (end 223.65 26.95) (width 0.3) (layer F.Cu) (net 1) (status 30))
 (segment (start 224.525326 24.331954) (end 224.625326 24.331954) (width 0.3) (layer B.Cu) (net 14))
 (segment (start 224.625326 24.331954) (end 226.95 26.656628) (width 0.3) (layer B.Cu) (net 14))
 (segment (start 226.95 26.656628) (end 226.95 26.75) (width 0.3) (layer B.Cu) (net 14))
 (via (at 226.95 26.75) (size 0.4) (drill 0.31) (layers F.Cu B.Cu) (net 14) (status 30))
 (via (at 224.525326 24.331954) (size 0.4) (drill 0.31) (layers F.Cu B.Cu) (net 14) (status 30))
 (segment (start 226.95 26.75) (end 226.95 27.45) (width 0.3) (layer F.Cu) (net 14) (status 10))
 (segment (start 226.95 27.45) (end 226.15 28.25) (width 0.3) (layer F.Cu) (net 14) (status 20))
 (segment (start 209.758309 29.144979) (end 206.998309 29.144979) (width 0.3) (layer F.Cu) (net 15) (status 30))
 (segment (start 206.998309 29.144979) (end 206.958309 29.184979) (width 0.3) (layer F.Cu) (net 15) (status 30))
 (segment (start 209.758309 26.644979) (end 206.958309 26.644979) (width 0.3) (layer F.Cu) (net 16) (status 30))
 (segment (start 209.758309 24.144979) (end 206.998309 24.144979) (width 0.3) (layer F.Cu) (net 17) (status 30))
 (segment (start 206.998309 24.144979) (end 206.958309 24.104979) (width 0.3) (layer F.Cu) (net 17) (status 30))
 (segment (start 206.958309 21.564979) (end 209.678309 21.564979) (width 0.3) (layer F.Cu) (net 18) (status 30))
 (segment (start 209.678309 21.564979) (end 209.758309 21.644979) (width 0.3) (layer F.Cu) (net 18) (status 30))
 (segment (start 226.025326 23.431954) (end 226.025326 21.268354) (width 0.3) (layer F.Cu) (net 19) (status 10))
 (segment (start 226.025326 21.268354) (end 225.688926 20.931954) (width 0.3) (layer F.Cu) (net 19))
 (segment (start 225.688926 20.931954) (end 224.525326 20.931954) (width 0.3) (layer F.Cu) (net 19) (status 20))
 (segment (start 224.525326 23.431954) (end 226.025326 23.431954) (width 0.3) (layer F.Cu) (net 19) (status 30))
 (segment (start 223.025326 23.431954) (end 223.025326 21.971954) (width 0.3) (layer F.Cu) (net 20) (status 10))
 (segment (start 223.025326 21.971954) (end 221.985326 20.931954) (width 0.3) (layer F.Cu) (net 20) (status 20))
 (segment (start 221.525326 23.431954) (end 223.025326 23.431954) (width 0.3) (layer F.Cu) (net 20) (status 30))
 (segment (start 220.025326 23.431954) (end 220.025326 21.511954) (width 0.3) (layer F.Cu) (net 21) (status 30))
 (segment (start 220.025326 21.511954) (end 219.445326 20.931954) (width 0.3) (layer F.Cu) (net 21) (status 30))
 (segment (start 218.525326 23.431954) (end 220.025326 23.431954) (width 0.3) (layer F.Cu) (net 21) (status 30))
 (segment (start 217.025326 23.431954) (end 217.025326 21.051954) (width 0.3) (layer F.Cu) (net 22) (status 30))
 (segment (start 217.025326 21.051954) (end 216.905326 20.931954) (width 0.3) (layer F.Cu) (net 22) (status 30))
 (segment (start 215.525326 23.431954) (end 217.025326 23.431954) (width 0.3) (layer F.Cu) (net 22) (status 30)))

